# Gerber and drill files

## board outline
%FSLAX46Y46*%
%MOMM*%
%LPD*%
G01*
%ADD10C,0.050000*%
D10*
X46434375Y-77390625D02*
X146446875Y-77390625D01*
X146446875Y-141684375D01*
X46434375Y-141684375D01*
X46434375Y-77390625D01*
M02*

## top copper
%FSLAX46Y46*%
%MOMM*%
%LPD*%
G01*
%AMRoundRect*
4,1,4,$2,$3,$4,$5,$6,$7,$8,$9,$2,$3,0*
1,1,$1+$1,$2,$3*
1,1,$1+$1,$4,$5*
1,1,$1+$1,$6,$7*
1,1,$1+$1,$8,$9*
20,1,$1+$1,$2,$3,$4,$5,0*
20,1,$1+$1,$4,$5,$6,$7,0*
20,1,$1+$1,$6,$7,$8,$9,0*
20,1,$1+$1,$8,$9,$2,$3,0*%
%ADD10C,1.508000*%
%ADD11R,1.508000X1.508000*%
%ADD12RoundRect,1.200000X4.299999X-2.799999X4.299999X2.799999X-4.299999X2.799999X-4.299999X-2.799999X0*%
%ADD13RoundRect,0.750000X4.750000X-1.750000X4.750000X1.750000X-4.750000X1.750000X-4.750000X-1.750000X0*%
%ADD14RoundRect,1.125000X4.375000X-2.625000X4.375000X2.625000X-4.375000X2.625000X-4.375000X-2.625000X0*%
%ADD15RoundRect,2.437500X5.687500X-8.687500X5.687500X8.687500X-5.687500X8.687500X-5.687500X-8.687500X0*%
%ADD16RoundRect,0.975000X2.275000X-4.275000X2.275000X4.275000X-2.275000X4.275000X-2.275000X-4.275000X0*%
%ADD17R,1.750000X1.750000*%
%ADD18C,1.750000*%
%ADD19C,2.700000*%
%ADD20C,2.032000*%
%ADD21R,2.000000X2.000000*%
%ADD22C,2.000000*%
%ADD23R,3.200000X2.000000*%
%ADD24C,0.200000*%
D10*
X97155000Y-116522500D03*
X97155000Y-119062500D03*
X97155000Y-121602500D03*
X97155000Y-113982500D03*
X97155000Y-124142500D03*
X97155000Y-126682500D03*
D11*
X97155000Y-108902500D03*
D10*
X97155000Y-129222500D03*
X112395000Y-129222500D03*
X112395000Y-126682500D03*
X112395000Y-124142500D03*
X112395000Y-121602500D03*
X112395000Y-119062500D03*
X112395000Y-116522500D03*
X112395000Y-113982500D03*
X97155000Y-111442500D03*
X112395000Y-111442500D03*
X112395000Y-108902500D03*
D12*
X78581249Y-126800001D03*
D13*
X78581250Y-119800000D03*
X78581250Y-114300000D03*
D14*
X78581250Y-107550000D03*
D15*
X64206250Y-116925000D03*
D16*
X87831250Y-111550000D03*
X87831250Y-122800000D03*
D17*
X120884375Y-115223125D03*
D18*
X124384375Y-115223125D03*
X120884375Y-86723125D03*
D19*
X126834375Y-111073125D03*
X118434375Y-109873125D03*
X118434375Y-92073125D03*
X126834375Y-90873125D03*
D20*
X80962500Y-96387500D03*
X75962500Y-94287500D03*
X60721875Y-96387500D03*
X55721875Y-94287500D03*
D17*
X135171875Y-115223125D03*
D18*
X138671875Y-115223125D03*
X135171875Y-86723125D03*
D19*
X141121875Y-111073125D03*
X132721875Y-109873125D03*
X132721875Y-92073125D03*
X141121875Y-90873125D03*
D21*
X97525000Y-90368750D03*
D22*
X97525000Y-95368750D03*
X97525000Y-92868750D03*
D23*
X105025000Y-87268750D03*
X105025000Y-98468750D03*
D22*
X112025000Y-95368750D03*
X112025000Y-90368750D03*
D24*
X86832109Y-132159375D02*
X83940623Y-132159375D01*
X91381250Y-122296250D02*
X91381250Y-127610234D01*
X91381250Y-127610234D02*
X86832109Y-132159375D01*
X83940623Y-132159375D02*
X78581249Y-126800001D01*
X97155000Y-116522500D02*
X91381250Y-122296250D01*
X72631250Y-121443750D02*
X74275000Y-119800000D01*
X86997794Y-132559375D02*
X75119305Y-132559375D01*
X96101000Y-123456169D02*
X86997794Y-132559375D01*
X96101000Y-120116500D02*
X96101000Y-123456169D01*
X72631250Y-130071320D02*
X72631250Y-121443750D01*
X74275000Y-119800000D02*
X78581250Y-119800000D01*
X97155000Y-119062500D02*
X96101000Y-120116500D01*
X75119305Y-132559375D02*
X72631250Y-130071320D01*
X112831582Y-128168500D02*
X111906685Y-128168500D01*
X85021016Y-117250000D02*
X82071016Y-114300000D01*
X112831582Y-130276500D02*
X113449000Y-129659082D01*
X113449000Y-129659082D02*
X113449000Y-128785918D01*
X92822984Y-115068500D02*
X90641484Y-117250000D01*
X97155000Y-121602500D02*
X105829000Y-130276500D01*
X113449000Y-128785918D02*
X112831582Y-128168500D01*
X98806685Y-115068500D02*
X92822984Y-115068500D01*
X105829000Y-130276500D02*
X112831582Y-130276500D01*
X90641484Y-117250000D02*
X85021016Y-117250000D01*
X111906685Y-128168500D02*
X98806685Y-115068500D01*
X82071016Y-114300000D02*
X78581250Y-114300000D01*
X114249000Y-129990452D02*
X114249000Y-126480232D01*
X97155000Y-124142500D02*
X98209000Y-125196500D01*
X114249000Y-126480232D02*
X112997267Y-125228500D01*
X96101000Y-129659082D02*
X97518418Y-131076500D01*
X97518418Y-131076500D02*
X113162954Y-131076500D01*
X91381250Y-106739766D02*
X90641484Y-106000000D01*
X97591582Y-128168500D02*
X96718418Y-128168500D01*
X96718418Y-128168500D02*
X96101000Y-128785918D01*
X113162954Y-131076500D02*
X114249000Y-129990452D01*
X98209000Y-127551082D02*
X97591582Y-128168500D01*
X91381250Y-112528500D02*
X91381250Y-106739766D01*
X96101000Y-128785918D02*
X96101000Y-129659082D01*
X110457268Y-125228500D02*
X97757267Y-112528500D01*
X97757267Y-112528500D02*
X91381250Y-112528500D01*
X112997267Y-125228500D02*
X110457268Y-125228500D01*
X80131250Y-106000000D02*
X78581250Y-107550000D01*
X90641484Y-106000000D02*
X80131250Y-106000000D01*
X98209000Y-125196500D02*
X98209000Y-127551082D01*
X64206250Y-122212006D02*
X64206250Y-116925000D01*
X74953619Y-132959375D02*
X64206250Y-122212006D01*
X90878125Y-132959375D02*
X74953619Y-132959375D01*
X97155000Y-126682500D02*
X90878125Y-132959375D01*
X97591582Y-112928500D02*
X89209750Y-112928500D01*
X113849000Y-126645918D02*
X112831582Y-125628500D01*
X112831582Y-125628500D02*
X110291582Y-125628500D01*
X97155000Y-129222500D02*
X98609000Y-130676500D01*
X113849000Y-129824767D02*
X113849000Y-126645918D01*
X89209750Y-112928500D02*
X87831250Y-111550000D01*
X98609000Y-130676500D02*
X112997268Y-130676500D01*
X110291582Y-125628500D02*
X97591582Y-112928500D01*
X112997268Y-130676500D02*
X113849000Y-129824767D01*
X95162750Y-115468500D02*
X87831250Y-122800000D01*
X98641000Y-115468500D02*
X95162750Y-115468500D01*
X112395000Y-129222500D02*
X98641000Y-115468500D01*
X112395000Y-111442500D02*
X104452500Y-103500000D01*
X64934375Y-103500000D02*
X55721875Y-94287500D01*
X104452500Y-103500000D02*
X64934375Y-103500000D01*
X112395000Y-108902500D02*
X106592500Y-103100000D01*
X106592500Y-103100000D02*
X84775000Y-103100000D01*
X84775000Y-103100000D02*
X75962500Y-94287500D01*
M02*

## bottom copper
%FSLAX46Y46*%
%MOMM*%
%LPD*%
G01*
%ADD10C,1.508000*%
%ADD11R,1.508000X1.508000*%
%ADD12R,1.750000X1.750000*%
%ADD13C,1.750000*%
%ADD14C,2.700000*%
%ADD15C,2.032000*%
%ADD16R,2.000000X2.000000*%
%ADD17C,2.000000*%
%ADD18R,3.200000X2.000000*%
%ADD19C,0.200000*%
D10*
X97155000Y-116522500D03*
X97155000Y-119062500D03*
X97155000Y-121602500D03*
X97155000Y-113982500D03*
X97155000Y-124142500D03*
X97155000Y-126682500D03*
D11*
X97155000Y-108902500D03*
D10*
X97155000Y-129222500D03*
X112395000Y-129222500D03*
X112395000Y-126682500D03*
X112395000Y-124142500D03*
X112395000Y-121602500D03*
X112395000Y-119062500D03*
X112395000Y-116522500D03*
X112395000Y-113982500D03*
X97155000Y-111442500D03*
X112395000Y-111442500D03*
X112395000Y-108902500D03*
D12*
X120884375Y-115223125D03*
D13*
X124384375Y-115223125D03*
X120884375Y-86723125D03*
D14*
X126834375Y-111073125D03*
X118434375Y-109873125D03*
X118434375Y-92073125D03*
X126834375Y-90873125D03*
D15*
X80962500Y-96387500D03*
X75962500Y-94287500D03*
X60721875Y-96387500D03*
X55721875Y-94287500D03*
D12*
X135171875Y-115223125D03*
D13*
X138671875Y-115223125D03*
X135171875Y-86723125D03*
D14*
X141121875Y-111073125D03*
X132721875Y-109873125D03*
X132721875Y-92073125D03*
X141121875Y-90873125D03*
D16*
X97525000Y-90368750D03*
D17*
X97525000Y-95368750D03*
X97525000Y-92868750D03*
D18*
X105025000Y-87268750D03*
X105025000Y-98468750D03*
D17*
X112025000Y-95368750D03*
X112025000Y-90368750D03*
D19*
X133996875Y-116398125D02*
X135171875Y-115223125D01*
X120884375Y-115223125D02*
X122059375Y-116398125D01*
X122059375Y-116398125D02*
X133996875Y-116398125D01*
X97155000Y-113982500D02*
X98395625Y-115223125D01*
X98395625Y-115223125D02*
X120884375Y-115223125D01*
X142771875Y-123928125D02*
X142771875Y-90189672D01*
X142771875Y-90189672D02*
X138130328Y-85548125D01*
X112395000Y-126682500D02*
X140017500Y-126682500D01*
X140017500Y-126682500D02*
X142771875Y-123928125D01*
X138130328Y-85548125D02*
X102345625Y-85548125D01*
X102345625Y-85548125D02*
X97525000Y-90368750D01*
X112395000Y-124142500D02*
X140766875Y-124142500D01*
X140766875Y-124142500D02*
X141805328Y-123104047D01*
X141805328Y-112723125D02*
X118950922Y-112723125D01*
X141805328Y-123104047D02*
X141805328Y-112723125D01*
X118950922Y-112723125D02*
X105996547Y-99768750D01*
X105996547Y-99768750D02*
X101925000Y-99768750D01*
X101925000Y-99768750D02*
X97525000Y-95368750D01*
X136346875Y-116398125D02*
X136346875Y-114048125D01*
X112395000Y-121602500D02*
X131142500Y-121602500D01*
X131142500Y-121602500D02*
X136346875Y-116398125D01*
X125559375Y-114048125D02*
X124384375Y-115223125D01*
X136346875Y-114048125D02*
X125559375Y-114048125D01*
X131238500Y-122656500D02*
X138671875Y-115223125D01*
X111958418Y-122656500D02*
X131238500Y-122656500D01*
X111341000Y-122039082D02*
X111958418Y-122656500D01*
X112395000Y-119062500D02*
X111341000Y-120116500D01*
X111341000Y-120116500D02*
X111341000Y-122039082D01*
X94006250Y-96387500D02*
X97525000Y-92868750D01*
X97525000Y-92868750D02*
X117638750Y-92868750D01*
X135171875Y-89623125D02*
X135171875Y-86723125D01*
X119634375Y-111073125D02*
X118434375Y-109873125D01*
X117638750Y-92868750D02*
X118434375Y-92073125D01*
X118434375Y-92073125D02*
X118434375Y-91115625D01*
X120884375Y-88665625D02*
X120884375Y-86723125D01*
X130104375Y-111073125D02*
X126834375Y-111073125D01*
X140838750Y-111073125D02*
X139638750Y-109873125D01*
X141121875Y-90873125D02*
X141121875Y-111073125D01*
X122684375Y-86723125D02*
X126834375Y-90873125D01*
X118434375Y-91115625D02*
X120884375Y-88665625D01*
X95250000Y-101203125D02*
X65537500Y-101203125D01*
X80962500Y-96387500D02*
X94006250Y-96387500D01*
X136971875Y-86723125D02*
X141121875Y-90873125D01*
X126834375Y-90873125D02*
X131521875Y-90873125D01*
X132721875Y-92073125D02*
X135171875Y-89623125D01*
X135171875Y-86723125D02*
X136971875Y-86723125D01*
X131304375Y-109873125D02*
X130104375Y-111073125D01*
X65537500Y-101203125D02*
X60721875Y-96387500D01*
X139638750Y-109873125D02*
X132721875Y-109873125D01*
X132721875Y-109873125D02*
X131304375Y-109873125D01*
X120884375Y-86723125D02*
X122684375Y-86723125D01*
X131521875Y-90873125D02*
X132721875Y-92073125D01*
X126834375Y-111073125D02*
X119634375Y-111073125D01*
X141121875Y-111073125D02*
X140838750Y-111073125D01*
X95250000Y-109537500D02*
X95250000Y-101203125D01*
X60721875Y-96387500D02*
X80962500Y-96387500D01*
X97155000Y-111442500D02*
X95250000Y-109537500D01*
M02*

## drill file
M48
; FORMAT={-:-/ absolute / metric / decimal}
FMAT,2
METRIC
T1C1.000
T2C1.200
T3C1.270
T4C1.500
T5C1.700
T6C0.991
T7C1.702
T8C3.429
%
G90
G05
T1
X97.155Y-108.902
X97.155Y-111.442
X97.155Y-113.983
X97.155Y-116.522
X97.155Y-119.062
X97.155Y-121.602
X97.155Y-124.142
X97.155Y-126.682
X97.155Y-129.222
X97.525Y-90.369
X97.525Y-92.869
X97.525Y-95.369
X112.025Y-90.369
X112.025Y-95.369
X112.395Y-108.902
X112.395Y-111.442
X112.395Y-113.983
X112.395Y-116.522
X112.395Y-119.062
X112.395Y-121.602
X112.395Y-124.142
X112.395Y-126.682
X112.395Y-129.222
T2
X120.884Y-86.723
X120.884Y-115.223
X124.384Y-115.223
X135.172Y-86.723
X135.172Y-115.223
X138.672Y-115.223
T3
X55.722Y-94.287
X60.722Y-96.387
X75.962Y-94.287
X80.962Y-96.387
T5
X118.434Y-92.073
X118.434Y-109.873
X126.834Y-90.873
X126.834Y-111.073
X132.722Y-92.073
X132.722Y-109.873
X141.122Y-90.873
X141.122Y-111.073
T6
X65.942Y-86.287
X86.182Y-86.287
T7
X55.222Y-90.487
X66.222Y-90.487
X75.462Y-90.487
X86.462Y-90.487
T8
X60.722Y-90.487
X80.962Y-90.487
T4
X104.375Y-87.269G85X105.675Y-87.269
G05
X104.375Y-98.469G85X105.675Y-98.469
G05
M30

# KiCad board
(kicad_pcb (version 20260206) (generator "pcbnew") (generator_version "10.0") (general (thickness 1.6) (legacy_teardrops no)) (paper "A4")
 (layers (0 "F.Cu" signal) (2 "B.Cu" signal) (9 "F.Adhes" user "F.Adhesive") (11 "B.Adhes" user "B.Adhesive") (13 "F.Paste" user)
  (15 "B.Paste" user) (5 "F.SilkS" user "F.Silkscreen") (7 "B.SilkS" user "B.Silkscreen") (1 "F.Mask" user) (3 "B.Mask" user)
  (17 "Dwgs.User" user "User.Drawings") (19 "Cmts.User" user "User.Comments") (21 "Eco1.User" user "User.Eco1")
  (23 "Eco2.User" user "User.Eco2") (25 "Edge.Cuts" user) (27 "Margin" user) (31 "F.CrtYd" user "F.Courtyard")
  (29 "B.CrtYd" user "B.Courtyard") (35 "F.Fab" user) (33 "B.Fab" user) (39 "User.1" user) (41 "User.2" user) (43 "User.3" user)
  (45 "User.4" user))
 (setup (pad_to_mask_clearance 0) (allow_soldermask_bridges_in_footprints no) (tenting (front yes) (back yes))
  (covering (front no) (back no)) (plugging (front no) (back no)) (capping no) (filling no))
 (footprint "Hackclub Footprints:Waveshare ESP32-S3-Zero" (layer "F.Cu") (at 104.775 119.0625)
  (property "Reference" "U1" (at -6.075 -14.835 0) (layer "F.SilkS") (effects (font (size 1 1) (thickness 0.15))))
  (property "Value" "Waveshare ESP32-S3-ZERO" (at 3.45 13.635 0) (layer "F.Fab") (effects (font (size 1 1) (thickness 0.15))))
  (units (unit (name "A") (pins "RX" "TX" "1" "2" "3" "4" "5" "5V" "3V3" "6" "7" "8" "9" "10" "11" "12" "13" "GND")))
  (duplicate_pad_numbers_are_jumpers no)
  (pad "1" thru_hole circle (at -7.62 -2.54) (size 1.508 1.508) (drill 1) (layers "*.Cu" "*.Mask") (remove_unused_layers no) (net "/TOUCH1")
   (solder_mask_margin 0.102))
  (pad "2" thru_hole circle (at -7.62 0) (size 1.508 1.508) (drill 1) (layers "*.Cu" "*.Mask") (remove_unused_layers no) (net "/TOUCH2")
   (solder_mask_margin 0.102))
  (pad "3" thru_hole circle (at -7.62 2.54) (size 1.508 1.508) (drill 1) (layers "*.Cu" "*.Mask") (remove_unused_layers no) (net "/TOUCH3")
   (solder_mask_margin 0.102))
  (pad "3V3" thru_hole circle (at -7.62 -5.08) (size 1.508 1.508) (drill 1) (layers "*.Cu" "*.Mask") (remove_unused_layers no) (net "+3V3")
   (solder_mask_margin 0.102))
  (pad "4" thru_hole circle (at -7.62 5.08) (size 1.508 1.508) (drill 1) (layers "*.Cu" "*.Mask") (remove_unused_layers no) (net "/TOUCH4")
   (solder_mask_margin 0.102))
  (pad "5" thru_hole circle (at -7.62 7.62) (size 1.508 1.508) (drill 1) (layers "*.Cu" "*.Mask") (remove_unused_layers no) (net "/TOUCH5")
   (solder_mask_margin 0.102))
  (pad "5V" thru_hole rect (at -7.62 -10.16) (size 1.508 1.508) (drill 1) (layers "*.Cu" "*.Mask") (remove_unused_layers no) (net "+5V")
   (solder_mask_margin 0.102))
  (pad "6" thru_hole circle (at -7.62 10.16) (size 1.508 1.508) (drill 1) (layers "*.Cu" "*.Mask") (remove_unused_layers no) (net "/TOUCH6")
   (solder_mask_margin 0.102))
  (pad "7" thru_hole circle (at 7.62 10.16) (size 1.508 1.508) (drill 1) (layers "*.Cu" "*.Mask") (remove_unused_layers no) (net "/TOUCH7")
   (solder_mask_margin 0.102))
  (pad "8" thru_hole circle (at 7.62 7.62) (size 1.508 1.508) (drill 1) (layers "*.Cu" "*.Mask") (remove_unused_layers no) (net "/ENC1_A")
   (solder_mask_margin 0.102))
  (pad "9" thru_hole circle (at 7.62 5.08) (size 1.508 1.508) (drill 1) (layers "*.Cu" "*.Mask") (remove_unused_layers no) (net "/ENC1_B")
   (solder_mask_margin 0.102))
  (pad "10" thru_hole circle (at 7.62 2.54) (size 1.508 1.508) (drill 1) (layers "*.Cu" "*.Mask") (remove_unused_layers no) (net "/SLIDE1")
   (solder_mask_margin 0.102))
  (pad "11" thru_hole circle (at 7.62 0) (size 1.508 1.508) (drill 1) (layers "*.Cu" "*.Mask") (remove_unused_layers no) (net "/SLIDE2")
   (solder_mask_margin 0.102))
  (pad "12" thru_hole circle (at 7.62 -2.54) (size 1.508 1.508) (drill 1) (layers "*.Cu" "*.Mask") (remove_unused_layers no)
   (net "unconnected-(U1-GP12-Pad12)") (solder_mask_margin 0.102))
  (pad "13" thru_hole circle (at 7.62 -5.08) (size 1.508 1.508) (drill 1) (layers "*.Cu" "*.Mask") (remove_unused_layers no)
   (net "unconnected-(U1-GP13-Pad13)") (solder_mask_margin 0.102))
  (pad "GND" thru_hole circle (at -7.62 -7.62) (size 1.508 1.508) (drill 1) (layers "*.Cu" "*.Mask") (remove_unused_layers no) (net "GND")
   (solder_mask_margin 0.102))
  (pad "RX" thru_hole circle (at 7.62 -7.62) (size 1.508 1.508) (drill 1) (layers "*.Cu" "*.Mask") (remove_unused_layers no)
   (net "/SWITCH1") (solder_mask_margin 0.102))
  (pad "TX" thru_hole circle (at 7.62 -10.16) (size 1.508 1.508) (drill 1) (layers "*.Cu" "*.Mask") (remove_unused_layers no)
   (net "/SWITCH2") (solder_mask_margin 0.102)))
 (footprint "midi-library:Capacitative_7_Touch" (layer "F.Cu") (at 48.20625 135.8 90)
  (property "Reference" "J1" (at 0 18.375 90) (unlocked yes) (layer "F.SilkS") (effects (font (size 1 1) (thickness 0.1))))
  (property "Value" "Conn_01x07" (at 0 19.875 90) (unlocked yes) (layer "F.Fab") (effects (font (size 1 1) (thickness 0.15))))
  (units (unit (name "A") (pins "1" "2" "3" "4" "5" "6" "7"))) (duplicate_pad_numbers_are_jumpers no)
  (pad "1" smd roundrect (at 8.999999 30.374999 90) (size 7.999998 10.999998) (layers "F.Cu" "F.Mask") (roundrect_rratio 0.15)
   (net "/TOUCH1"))
  (pad "2" smd roundrect (at 16 30.375 90) (size 5 11) (layers "F.Cu" "F.Mask") (roundrect_rratio 0.15) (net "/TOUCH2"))
  (pad "3" smd roundrect (at 21.5 30.375 90) (size 5 11) (layers "F.Cu" "F.Mask") (roundrect_rratio 0.15) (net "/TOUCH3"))
  (pad "4" smd roundrect (at 28.25 30.375 90) (size 7.5 11) (layers "F.Cu" "F.Mask") (roundrect_rratio 0.15) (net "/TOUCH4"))
  (pad "5" smd roundrect (at 18.875 16 90) (size 22.25 16.25) (layers "F.Cu" "F.Mask") (roundrect_rratio 0.15) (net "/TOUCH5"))
  (pad "6" smd roundrect (at 24.25 39.625 90) (size 10.5 6.5) (layers "F.Cu" "F.Mask") (roundrect_rratio 0.15) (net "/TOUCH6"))
  (pad "7" smd roundrect (at 13 39.625 90) (size 10.5 6.5) (layers "F.Cu" "F.Mask") (roundrect_rratio 0.15) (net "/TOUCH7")))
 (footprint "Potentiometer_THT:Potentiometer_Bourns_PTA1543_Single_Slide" (layer "F.Cu") (at 120.884375 115.223125 90)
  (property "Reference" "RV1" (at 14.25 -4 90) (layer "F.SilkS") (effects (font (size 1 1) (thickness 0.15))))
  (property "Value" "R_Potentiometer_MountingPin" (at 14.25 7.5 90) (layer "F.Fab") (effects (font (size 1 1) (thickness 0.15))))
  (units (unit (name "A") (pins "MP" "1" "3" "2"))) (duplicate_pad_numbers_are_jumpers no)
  (pad "1" thru_hole rect (at 0 0 90) (size 1.75 1.75) (drill 1.2) (layers "*.Cu" "*.Mask") (remove_unused_layers no) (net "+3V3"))
  (pad "2" thru_hole circle (at 0 3.5 90) (size 1.75 1.75) (drill 1.2) (layers "*.Cu" "*.Mask") (remove_unused_layers no) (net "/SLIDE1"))
  (pad "3" thru_hole circle (at 28.5 0 90) (size 1.75 1.75) (drill 1.2) (layers "*.Cu" "*.Mask") (remove_unused_layers no) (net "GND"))
  (pad "MP" thru_hole circle (at 4.15 5.95 90) (size 2.7 2.7) (drill 1.7) (layers "*.Cu" "*.Mask") (remove_unused_layers no) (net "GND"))
  (pad "MP" thru_hole circle (at 5.35 -2.45 90) (size 2.7 2.7) (drill 1.7) (layers "*.Cu" "*.Mask") (remove_unused_layers no) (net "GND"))
  (pad "MP" thru_hole circle (at 23.15 -2.45 90) (size 2.7 2.7) (drill 1.7) (layers "*.Cu" "*.Mask") (remove_unused_layers no) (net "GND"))
  (pad "MP" thru_hole circle (at 24.35 5.95 90) (size 2.7 2.7) (drill 1.7) (layers "*.Cu" "*.Mask") (remove_unused_layers no) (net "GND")))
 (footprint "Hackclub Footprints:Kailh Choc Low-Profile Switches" (layer "F.Cu") (at 80.9625 90.4875)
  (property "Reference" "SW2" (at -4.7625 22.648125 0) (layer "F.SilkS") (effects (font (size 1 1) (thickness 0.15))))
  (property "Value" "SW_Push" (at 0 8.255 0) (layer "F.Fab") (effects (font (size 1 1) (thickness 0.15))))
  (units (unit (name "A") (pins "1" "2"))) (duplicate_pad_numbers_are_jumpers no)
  (pad "" np_thru_hole circle (at -5.5 0) (size 1.7018 1.7018) (drill 1.7018) (layers "*.Cu" "*.Mask"))
  (pad "" np_thru_hole circle (at 0 0) (size 3.429 3.429) (drill 3.429) (layers "*.Cu" "*.Mask"))
  (pad "" np_thru_hole circle (at 5.22 -4.2) (size 0.9906 0.9906) (drill 0.9906) (layers "*.Cu" "*.Mask"))
  (pad "" np_thru_hole circle (at 5.5 0) (size 1.7018 1.7018) (drill 1.7018) (layers "*.Cu" "*.Mask"))
  (pad "1" thru_hole circle (at 0 5.9) (size 2.032 2.032) (drill 1.27) (layers "*.Cu" "*.Mask") (remove_unused_layers no) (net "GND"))
  (pad "2" thru_hole circle (at -5 3.8) (size 2.032 2.032) (drill 1.27) (layers "*.Cu" "*.Mask") (remove_unused_layers no) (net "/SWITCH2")))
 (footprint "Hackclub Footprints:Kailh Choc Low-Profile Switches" (layer "F.Cu") (at 60.721875 90.4875)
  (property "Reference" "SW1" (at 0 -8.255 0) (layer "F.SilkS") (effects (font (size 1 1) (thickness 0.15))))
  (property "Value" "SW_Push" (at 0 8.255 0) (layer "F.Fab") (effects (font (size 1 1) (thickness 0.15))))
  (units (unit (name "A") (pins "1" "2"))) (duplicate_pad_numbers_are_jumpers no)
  (pad "" np_thru_hole circle (at -5.5 0) (size 1.7018 1.7018) (drill 1.7018) (layers "*.Cu" "*.Mask"))
  (pad "" np_thru_hole circle (at 0 0) (size 3.429 3.429) (drill 3.429) (layers "*.Cu" "*.Mask"))
  (pad "" np_thru_hole circle (at 5.22 -4.2) (size 0.9906 0.9906) (drill 0.9906) (layers "*.Cu" "*.Mask"))
  (pad "" np_thru_hole circle (at 5.5 0) (size 1.7018 1.7018) (drill 1.7018) (layers "*.Cu" "*.Mask"))
  (pad "1" thru_hole circle (at 0 5.9) (size 2.032 2.032) (drill 1.27) (layers "*.Cu" "*.Mask") (remove_unused_layers no) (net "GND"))
  (pad "2" thru_hole circle (at -5 3.8) (size 2.032 2.032) (drill 1.27) (layers "*.Cu" "*.Mask") (remove_unused_layers no) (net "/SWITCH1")))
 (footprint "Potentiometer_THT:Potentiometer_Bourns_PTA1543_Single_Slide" (layer "F.Cu") (at 135.171875 115.223125 90)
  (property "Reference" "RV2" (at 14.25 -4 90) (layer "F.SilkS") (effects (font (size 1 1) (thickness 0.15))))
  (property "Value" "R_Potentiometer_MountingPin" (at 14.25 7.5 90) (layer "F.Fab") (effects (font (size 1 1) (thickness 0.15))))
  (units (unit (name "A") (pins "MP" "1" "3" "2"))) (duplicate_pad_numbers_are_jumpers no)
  (pad "1" thru_hole rect (at 0 0 90) (size 1.75 1.75) (drill 1.2) (layers "*.Cu" "*.Mask") (remove_unused_layers no) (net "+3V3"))
  (pad "2" thru_hole circle (at 0 3.5 90) (size 1.75 1.75) (drill 1.2) (layers "*.Cu" "*.Mask") (remove_unused_layers no) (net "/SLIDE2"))
  (pad "3" thru_hole circle (at 28.5 0 90) (size 1.75 1.75) (drill 1.2) (layers "*.Cu" "*.Mask") (remove_unused_layers no) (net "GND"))
  (pad "MP" thru_hole circle (at 4.15 5.95 90) (size 2.7 2.7) (drill 1.7) (layers "*.Cu" "*.Mask") (remove_unused_layers no) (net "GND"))
  (pad "MP" thru_hole circle (at 5.35 -2.45 90) (size 2.7 2.7) (drill 1.7) (layers "*.Cu" "*.Mask") (remove_unused_layers no) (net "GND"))
  (pad "MP" thru_hole circle (at 23.15 -2.45 90) (size 2.7 2.7) (drill 1.7) (layers "*.Cu" "*.Mask") (remove_unused_layers no) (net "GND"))
  (pad "MP" thru_hole circle (at 24.35 5.95 90) (size 2.7 2.7) (drill 1.7) (layers "*.Cu" "*.Mask") (remove_unused_layers no) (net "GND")))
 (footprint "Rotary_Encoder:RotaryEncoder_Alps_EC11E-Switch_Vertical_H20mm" (layer "F.Cu") (at 97.525 90.36875)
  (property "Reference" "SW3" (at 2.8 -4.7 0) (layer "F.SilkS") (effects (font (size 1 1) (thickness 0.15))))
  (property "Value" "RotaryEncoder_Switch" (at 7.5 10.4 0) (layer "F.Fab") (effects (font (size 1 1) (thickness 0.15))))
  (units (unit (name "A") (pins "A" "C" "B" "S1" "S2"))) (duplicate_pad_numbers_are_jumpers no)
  (pad "A" thru_hole rect (at 0 0) (size 2 2) (drill 1) (layers "*.Cu" "*.Mask") (remove_unused_layers no) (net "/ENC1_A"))
  (pad "B" thru_hole circle (at 0 5) (size 2 2) (drill 1) (layers "*.Cu" "*.Mask") (remove_unused_layers no) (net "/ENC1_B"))
  (pad "C" thru_hole circle (at 0 2.5) (size 2 2) (drill 1) (layers "*.Cu" "*.Mask") (remove_unused_layers no) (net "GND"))
  (pad "MP" thru_hole rect (at 7.5 -3.1) (size 3.2 2) (drill oval 2.8 1.5) (layers "*.Cu" "*.Mask") (remove_unused_layers no))
  (pad "MP" thru_hole rect (at 7.5 8.1) (size 3.2 2) (drill oval 2.8 1.5) (layers "*.Cu" "*.Mask") (remove_unused_layers no))
  (pad "S1" thru_hole circle (at 14.5 5) (size 2 2) (drill 1) (layers "*.Cu" "*.Mask") (remove_unused_layers no)
   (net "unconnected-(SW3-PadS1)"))
  (pad "S2" thru_hole circle (at 14.5 0) (size 2 2) (drill 1) (layers "*.Cu" "*.Mask") (remove_unused_layers no)
   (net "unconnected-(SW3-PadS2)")))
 (gr_rect (start 46.434375 77.390625) (end 146.446875 141.684375) (stroke (width 0.05) (type default)) (fill no) (layer "Edge.Cuts"))
 (segment (start 86.832109 132.159375) (end 83.940623 132.159375) (width 0.2) (layer "F.Cu") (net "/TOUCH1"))
 (segment (start 91.38125 122.29625) (end 91.38125 127.610234) (width 0.2) (layer "F.Cu") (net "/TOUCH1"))
 (segment (start 91.38125 127.610234) (end 86.832109 132.159375) (width 0.2) (layer "F.Cu") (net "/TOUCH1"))
 (segment (start 83.940623 132.159375) (end 78.581249 126.800001) (width 0.2) (layer "F.Cu") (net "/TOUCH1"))
 (segment (start 97.155 116.5225) (end 91.38125 122.29625) (width 0.2) (layer "F.Cu") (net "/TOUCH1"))
 (segment (start 72.63125 121.44375) (end 74.275 119.8) (width 0.2) (layer "F.Cu") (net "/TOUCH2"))
 (segment (start 86.997794 132.559375) (end 75.119305 132.559375) (width 0.2) (layer "F.Cu") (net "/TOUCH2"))
 (segment (start 96.101 123.456169) (end 86.997794 132.559375) (width 0.2) (layer "F.Cu") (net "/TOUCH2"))
 (segment (start 96.101 120.1165) (end 96.101 123.456169) (width 0.2) (layer "F.Cu") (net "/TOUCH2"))
 (segment (start 72.63125 130.07132) (end 72.63125 121.44375) (width 0.2) (layer "F.Cu") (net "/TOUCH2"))
 (segment (start 74.275 119.8) (end 78.58125 119.8) (width 0.2) (layer "F.Cu") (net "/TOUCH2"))
 (segment (start 97.155 119.0625) (end 96.101 120.1165) (width 0.2) (layer "F.Cu") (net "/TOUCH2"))
 (segment (start 75.119305 132.559375) (end 72.63125 130.07132) (width 0.2) (layer "F.Cu") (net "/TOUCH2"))
 (segment (start 112.831582 128.1685) (end 111.906685 128.1685) (width 0.2) (layer "F.Cu") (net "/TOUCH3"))
 (segment (start 85.021016 117.25) (end 82.071016 114.3) (width 0.2) (layer "F.Cu") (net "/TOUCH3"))
 (segment (start 112.831582 130.2765) (end 113.449 129.659082) (width 0.2) (layer "F.Cu") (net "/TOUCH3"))
 (segment (start 113.449 129.659082) (end 113.449 128.785918) (width 0.2) (layer "F.Cu") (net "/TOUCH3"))
 (segment (start 92.822984 115.0685) (end 90.641484 117.25) (width 0.2) (layer "F.Cu") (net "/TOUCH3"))
 (segment (start 97.155 121.6025) (end 105.829 130.2765) (width 0.2) (layer "F.Cu") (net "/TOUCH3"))
 (segment (start 113.449 128.785918) (end 112.831582 128.1685) (width 0.2) (layer "F.Cu") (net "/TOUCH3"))
 (segment (start 98.806685 115.0685) (end 92.822984 115.0685) (width 0.2) (layer "F.Cu") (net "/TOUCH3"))
 (segment (start 105.829 130.2765) (end 112.831582 130.2765) (width 0.2) (layer "F.Cu") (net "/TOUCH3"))
 (segment (start 90.641484 117.25) (end 85.021016 117.25) (width 0.2) (layer "F.Cu") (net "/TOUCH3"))
 (segment (start 111.906685 128.1685) (end 98.806685 115.0685) (width 0.2) (layer "F.Cu") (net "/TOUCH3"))
 (segment (start 82.071016 114.3) (end 78.58125 114.3) (width 0.2) (layer "F.Cu") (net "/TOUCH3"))
 (segment (start 133.996875 116.398125) (end 135.171875 115.223125) (width 0.2) (layer "B.Cu") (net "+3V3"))
 (segment (start 120.884375 115.223125) (end 122.059375 116.398125) (width 0.2) (layer "B.Cu") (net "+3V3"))
 (segment (start 122.059375 116.398125) (end 133.996875 116.398125) (width 0.2) (layer "B.Cu") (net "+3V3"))
 (segment (start 97.155 113.9825) (end 98.395625 115.223125) (width 0.2) (layer "B.Cu") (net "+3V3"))
 (segment (start 98.395625 115.223125) (end 120.884375 115.223125) (width 0.2) (layer "B.Cu") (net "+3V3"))
 (segment (start 114.249 129.990452) (end 114.249 126.480232) (width 0.2) (layer "F.Cu") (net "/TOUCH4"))
 (segment (start 97.155 124.1425) (end 98.209 125.1965) (width 0.2) (layer "F.Cu") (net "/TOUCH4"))
 (segment (start 114.249 126.480232) (end 112.997267 125.2285) (width 0.2) (layer "F.Cu") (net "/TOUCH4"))
 (segment (start 96.101 129.659082) (end 97.518418 131.0765) (width 0.2) (layer "F.Cu") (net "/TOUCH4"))
 (segment (start 97.518418 131.0765) (end 113.162954 131.0765) (width 0.2) (layer "F.Cu") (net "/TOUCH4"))
 (segment (start 91.38125 106.739766) (end 90.641484 106) (width 0.2) (layer "F.Cu") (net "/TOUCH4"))
 (segment (start 97.591582 128.1685) (end 96.718418 128.1685) (width 0.2) (layer "F.Cu") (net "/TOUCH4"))
 (segment (start 96.718418 128.1685) (end 96.101 128.785918) (width 0.2) (layer "F.Cu") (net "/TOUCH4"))
 (segment (start 113.162954 131.0765) (end 114.249 129.990452) (width 0.2) (layer "F.Cu") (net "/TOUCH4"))
 (segment (start 98.209 127.551082) (end 97.591582 128.1685) (width 0.2) (layer "F.Cu") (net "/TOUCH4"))
 (segment (start 91.38125 112.5285) (end 91.38125 106.739766) (width 0.2) (layer "F.Cu") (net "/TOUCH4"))
 (segment (start 96.101 128.785918) (end 96.101 129.659082) (width 0.2) (layer "F.Cu") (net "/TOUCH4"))
 (segment (start 110.457268 125.2285) (end 97.757267 112.5285) (width 0.2) (layer "F.Cu") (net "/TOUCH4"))
 (segment (start 97.757267 112.5285) (end 91.38125 112.5285) (width 0.2) (layer "F.Cu") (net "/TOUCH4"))
 (segment (start 112.997267 125.2285) (end 110.457268 125.2285) (width 0.2) (layer "F.Cu") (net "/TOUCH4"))
 (segment (start 80.13125 106) (end 78.58125 107.55) (width 0.2) (layer "F.Cu") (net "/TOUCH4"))
 (segment (start 90.641484 106) (end 80.13125 106) (width 0.2) (layer "F.Cu") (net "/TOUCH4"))
 (segment (start 98.209 125.1965) (end 98.209 127.551082) (width 0.2) (layer "F.Cu") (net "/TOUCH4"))
 (segment (start 64.20625 122.212006) (end 64.20625 116.925) (width 0.2) (layer "F.Cu") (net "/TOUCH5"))
 (segment (start 74.953619 132.959375) (end 64.20625 122.212006) (width 0.2) (layer "F.Cu") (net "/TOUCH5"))
 (segment (start 90.878125 132.959375) (end 74.953619 132.959375) (width 0.2) (layer "F.Cu") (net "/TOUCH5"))
 (segment (start 97.155 126.6825) (end 90.878125 132.959375) (width 0.2) (layer "F.Cu") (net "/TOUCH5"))
 (segment (start 97.591582 112.9285) (end 89.20975 112.9285) (width 0.2) (layer "F.Cu") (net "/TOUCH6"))
 (segment (start 113.849 126.645918) (end 112.831582 125.6285) (width 0.2) (layer "F.Cu") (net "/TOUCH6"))
 (segment (start 112.831582 125.6285) (end 110.291582 125.6285) (width 0.2) (layer "F.Cu") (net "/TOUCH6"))
 (segment (start 97.155 129.2225) (end 98.609 130.6765) (width 0.2) (layer "F.Cu") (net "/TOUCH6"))
 (segment (start 113.849 129.824767) (end 113.849 126.645918) (width 0.2) (layer "F.Cu") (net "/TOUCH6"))
 (segment (start 89.20975 112.9285) (end 87.83125 111.55) (width 0.2) (layer "F.Cu") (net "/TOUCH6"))
 (segment (start 98.609 130.6765) (end 112.997268 130.6765) (width 0.2) (layer "F.Cu") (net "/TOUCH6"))
 (segment (start 110.291582 125.6285) (end 97.591582 112.9285) (width 0.2) (layer "F.Cu") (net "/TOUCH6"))
 (segment (start 112.997268 130.6765) (end 113.849 129.824767) (width 0.2) (layer "F.Cu") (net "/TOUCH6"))
 (segment (start 95.16275 115.4685) (end 87.83125 122.8) (width 0.2) (layer "F.Cu") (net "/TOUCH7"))
 (segment (start 98.641 115.4685) (end 95.16275 115.4685) (width 0.2) (layer "F.Cu") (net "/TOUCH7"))
 (segment (start 112.395 129.2225) (end 98.641 115.4685) (width 0.2) (layer "F.Cu") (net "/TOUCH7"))
 (segment (start 142.771875 123.928125) (end 142.771875 90.189672) (width 0.2) (layer "B.Cu") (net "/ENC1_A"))
 (segment (start 142.771875 90.189672) (end 138.130328 85.548125) (width 0.2) (layer "B.Cu") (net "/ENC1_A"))
 (segment (start 112.395 126.6825) (end 140.0175 126.6825) (width 0.2) (layer "B.Cu") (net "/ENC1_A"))
 (segment (start 140.0175 126.6825) (end 142.771875 123.928125) (width 0.2) (layer "B.Cu") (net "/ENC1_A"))
 (segment (start 138.130328 85.548125) (end 102.345625 85.548125) (width 0.2) (layer "B.Cu") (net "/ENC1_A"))
 (segment (start 102.345625 85.548125) (end 97.525 90.36875) (width 0.2) (layer "B.Cu") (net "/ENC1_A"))
 (segment (start 112.395 124.1425) (end 140.766875 124.1425) (width 0.2) (layer "B.Cu") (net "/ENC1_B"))
 (segment (start 140.766875 124.1425) (end 141.805328 123.104047) (width 0.2) (layer "B.Cu") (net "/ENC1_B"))
 (segment (start 141.805328 112.723125) (end 118.950922 112.723125) (width 0.2) (layer "B.Cu") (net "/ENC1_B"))
 (segment (start 141.805328 123.104047) (end 141.805328 112.723125) (width 0.2) (layer "B.Cu") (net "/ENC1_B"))
 (segment (start 118.950922 112.723125) (end 105.996547 99.76875) (width 0.2) (layer "B.Cu") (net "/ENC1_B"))
 (segment (start 105.996547 99.76875) (end 101.925 99.76875) (width 0.2) (layer "B.Cu") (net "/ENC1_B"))
 (segment (start 101.925 99.76875) (end 97.525 95.36875) (width 0.2) (layer "B.Cu") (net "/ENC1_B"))
 (segment (start 136.346875 116.398125) (end 136.346875 114.048125) (width 0.2) (layer "B.Cu") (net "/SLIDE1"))
 (segment (start 112.395 121.6025) (end 131.1425 121.6025) (width 0.2) (layer "B.Cu") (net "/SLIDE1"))
 (segment (start 131.1425 121.6025) (end 136.346875 116.398125) (width 0.2) (layer "B.Cu") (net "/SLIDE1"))
 (segment (start 125.559375 114.048125) (end 124.384375 115.223125) (width 0.2) (layer "B.Cu") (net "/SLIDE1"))
 (segment (start 136.346875 114.048125) (end 125.559375 114.048125) (width 0.2) (layer "B.Cu") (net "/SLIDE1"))
 (segment (start 131.2385 122.6565) (end 138.671875 115.223125) (width 0.2) (layer "B.Cu") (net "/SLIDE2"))
 (segment (start 111.958418 122.6565) (end 131.2385 122.6565) (width 0.2) (layer "B.Cu") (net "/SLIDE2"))
 (segment (start 111.341 122.039082) (end 111.958418 122.6565) (width 0.2) (layer "B.Cu") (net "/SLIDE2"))
 (segment (start 112.395 119.0625) (end 111.341 120.1165) (width 0.2) (layer "B.Cu") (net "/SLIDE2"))
 (segment (start 111.341 120.1165) (end 111.341 122.039082) (width 0.2) (layer "B.Cu") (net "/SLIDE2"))
 (segment (start 94.00625 96.3875) (end 97.525 92.86875) (width 0.2) (layer "B.Cu") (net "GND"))
 (segment (start 97.525 92.86875) (end 117.63875 92.86875) (width 0.2) (layer "B.Cu") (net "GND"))
 (segment (start 135.171875 89.623125) (end 135.171875 86.723125) (width 0.2) (layer "B.Cu") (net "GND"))
 (segment (start 119.634375 111.073125) (end 118.434375 109.873125) (width 0.2) (layer "B.Cu") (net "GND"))
 (segment (start 117.63875 92.86875) (end 118.434375 92.073125) (width 0.2) (layer "B.Cu") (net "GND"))
 (segment (start 118.434375 92.073125) (end 118.434375 91.115625) (width 0.2) (layer "B.Cu") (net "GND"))
 (segment (start 120.884375 88.665625) (end 120.884375 86.723125) (width 0.2) (layer "B.Cu") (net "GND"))
 (segment (start 130.104375 111.073125) (end 126.834375 111.073125) (width 0.2) (layer "B.Cu") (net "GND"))
 (segment (start 140.83875 111.073125) (end 139.63875 109.873125) (width 0.2) (layer "B.Cu") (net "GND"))
 (segment (start 141.121875 90.873125) (end 141.121875 111.073125) (width 0.2) (layer "B.Cu") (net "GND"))
 (segment (start 122.684375 86.723125) (end 126.834375 90.873125) (width 0.2) (layer "B.Cu") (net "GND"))
 (segment (start 118.434375 91.115625) (end 120.884375 88.665625) (width 0.2) (layer "B.Cu") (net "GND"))
 (segment (start 95.25 101.203125) (end 65.5375 101.203125) (width 0.2) (layer "B.Cu") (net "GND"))
 (segment (start 80.9625 96.3875) (end 94.00625 96.3875) (width 0.2) (layer "B.Cu") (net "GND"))
 (segment (start 136.971875 86.723125) (end 141.121875 90.873125) (width 0.2) (layer "B.Cu") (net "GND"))
 (segment (start 126.834375 90.873125) (end 131.521875 90.873125) (width 0.2) (layer "B.Cu") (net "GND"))
 (segment (start 132.721875 92.073125) (end 135.171875 89.623125) (width 0.2) (layer "B.Cu") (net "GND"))
 (segment (start 135.171875 86.723125) (end 136.971875 86.723125) (width 0.2) (layer "B.Cu") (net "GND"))
 (segment (start 131.304375 109.873125) (end 130.104375 111.073125) (width 0.2) (layer "B.Cu") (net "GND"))
 (segment (start 65.5375 101.203125) (end 60.721875 96.3875) (width 0.2) (layer "B.Cu") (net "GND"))
 (segment (start 139.63875 109.873125) (end 132.721875 109.873125) (width 0.2) (layer "B.Cu") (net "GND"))
 (segment (start 132.721875 109.873125) (end 131.304375 109.873125) (width 0.2) (layer "B.Cu") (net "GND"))
 (segment (start 120.884375 86.723125) (end 122.684375 86.723125) (width 0.2) (layer "B.Cu") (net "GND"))
 (segment (start 131.521875 90.873125) (end 132.721875 92.073125) (width 0.2) (layer "B.Cu") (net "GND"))
 (segment (start 126.834375 111.073125) (end 119.634375 111.073125) (width 0.2) (layer "B.Cu") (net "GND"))
 (segment (start 141.121875 111.073125) (end 140.83875 111.073125) (width 0.2) (layer "B.Cu") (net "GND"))
 (segment (start 95.25 109.5375) (end 95.25 101.203125) (width 0.2) (layer "B.Cu") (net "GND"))
 (segment (start 60.721875 96.3875) (end 80.9625 96.3875) (width 0.2) (layer "B.Cu") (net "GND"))
 (segment (start 97.155 111.4425) (end 95.25 109.5375) (width 0.2) (layer "B.Cu") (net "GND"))
 (segment (start 112.395 111.4425) (end 104.4525 103.5) (width 0.2) (layer "F.Cu") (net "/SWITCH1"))
 (segment (start 64.934375 103.5) (end 55.721875 94.2875) (width 0.2) (layer "F.Cu") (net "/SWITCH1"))
 (segment (start 104.4525 103.5) (end 64.934375 103.5) (width 0.2) (layer "F.Cu") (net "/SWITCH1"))
 (segment (start 112.395 108.9025) (end 106.5925 103.1) (width 0.2) (layer "F.Cu") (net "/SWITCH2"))
 (segment (start 106.5925 103.1) (end 84.775 103.1) (width 0.2) (layer "F.Cu") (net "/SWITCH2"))
 (segment (start 84.775 103.1) (end 75.9625 94.2875) (width 0.2) (layer "F.Cu") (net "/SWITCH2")))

